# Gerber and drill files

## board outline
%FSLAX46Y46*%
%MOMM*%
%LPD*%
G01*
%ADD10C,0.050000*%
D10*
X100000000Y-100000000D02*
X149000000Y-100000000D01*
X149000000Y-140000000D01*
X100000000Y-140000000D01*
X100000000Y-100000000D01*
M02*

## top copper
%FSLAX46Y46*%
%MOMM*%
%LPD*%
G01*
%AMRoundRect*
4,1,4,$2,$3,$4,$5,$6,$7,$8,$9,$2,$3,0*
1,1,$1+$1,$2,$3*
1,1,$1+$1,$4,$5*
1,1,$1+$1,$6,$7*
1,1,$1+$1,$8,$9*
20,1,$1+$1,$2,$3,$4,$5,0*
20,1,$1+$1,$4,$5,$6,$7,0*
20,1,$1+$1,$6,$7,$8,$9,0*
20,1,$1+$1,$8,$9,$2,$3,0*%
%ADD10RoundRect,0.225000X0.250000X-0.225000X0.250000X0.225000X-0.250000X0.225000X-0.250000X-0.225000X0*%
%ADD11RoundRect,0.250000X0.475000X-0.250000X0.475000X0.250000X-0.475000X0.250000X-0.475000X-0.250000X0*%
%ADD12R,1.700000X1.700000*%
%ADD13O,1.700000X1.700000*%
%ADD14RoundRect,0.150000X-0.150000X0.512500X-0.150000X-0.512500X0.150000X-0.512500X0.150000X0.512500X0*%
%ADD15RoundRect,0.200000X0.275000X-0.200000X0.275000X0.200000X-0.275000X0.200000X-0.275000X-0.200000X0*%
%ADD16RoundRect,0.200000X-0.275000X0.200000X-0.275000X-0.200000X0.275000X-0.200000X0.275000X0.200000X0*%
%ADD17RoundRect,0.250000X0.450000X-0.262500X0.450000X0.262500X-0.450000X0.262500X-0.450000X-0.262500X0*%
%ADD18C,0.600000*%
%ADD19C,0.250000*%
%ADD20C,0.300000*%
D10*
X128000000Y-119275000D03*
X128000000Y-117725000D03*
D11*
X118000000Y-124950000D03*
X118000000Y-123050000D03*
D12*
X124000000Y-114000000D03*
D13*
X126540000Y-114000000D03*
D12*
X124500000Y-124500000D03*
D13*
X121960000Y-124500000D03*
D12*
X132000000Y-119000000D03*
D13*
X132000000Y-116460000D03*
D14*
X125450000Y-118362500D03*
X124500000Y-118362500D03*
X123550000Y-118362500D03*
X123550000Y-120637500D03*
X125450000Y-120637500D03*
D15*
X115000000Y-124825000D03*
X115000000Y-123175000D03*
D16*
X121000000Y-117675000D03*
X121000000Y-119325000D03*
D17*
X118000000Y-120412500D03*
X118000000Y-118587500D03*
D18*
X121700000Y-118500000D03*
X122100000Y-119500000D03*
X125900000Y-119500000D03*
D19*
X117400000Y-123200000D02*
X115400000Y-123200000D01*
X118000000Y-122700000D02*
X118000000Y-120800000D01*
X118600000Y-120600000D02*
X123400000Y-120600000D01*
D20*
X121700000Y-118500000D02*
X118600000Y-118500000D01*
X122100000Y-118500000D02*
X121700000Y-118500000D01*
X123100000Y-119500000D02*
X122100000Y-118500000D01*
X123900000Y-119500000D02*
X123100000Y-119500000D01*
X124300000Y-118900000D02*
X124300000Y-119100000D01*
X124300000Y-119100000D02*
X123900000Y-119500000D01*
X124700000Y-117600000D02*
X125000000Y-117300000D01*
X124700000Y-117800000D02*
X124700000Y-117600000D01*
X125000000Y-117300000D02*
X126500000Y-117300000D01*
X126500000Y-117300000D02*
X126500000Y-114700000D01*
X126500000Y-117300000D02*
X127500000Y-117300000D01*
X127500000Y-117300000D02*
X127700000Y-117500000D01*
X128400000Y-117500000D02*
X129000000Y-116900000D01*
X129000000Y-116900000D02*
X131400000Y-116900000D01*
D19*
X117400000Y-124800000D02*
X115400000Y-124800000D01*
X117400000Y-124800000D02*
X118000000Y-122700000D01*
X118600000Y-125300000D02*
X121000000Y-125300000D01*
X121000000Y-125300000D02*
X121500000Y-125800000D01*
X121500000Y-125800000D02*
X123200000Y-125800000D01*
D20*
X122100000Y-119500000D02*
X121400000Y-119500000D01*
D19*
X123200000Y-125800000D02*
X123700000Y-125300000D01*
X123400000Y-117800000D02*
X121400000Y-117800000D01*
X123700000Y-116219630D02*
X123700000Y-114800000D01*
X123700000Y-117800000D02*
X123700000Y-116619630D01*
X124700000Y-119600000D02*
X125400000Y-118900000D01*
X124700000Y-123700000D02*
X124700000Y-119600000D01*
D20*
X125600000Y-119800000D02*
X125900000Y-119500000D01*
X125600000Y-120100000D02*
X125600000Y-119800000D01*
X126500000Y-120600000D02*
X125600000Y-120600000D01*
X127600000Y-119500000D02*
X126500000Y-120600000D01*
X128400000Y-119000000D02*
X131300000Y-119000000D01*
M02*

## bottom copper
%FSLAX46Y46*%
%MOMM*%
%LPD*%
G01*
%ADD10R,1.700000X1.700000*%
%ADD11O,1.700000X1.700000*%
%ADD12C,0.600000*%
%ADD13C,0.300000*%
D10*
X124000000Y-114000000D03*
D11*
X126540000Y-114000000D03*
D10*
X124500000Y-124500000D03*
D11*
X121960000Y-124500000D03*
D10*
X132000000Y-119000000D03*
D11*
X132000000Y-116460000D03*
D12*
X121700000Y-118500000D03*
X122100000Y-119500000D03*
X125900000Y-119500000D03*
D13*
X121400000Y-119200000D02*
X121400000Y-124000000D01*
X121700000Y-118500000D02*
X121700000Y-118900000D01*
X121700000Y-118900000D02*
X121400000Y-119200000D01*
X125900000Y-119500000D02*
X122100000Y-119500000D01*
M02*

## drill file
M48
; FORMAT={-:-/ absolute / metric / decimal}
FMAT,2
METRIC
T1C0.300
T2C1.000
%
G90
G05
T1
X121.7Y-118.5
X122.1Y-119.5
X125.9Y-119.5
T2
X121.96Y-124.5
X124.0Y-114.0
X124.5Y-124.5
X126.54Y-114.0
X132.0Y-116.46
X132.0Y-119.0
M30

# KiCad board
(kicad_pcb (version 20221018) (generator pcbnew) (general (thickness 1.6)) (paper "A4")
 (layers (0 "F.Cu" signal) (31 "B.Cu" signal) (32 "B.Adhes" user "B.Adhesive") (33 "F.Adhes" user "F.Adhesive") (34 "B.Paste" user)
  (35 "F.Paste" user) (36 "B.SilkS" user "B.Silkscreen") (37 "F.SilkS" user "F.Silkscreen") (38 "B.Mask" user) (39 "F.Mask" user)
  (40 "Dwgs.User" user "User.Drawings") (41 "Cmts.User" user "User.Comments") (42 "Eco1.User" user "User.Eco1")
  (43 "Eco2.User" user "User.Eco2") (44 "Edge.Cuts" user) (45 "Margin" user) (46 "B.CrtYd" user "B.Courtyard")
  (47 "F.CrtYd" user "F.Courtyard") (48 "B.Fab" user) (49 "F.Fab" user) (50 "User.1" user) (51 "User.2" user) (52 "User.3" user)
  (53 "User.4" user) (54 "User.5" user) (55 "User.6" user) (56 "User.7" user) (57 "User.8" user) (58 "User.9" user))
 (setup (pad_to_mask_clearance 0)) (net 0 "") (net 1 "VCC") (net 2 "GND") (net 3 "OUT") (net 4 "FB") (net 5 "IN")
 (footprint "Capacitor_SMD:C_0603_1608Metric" (layer "F.Cu") (at 128 118.5 90)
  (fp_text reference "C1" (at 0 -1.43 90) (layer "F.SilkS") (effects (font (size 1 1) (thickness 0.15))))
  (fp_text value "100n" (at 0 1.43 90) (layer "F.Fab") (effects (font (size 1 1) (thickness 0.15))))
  (pad "1" smd roundrect (at -0.775 0 90) (size 0.9 0.95) (layers "F.Cu" "F.Paste" "F.Mask") (roundrect_rratio 0.25) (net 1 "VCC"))
  (pad "2" smd roundrect (at 0.775 0 90) (size 0.9 0.95) (layers "F.Cu" "F.Paste" "F.Mask") (roundrect_rratio 0.25) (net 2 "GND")))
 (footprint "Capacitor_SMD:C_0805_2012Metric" (layer "F.Cu") (at 118 124 90)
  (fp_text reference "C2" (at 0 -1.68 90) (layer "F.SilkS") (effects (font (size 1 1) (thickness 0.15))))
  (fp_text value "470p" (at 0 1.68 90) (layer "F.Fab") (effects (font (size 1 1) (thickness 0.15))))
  (pad "1" smd roundrect (at -0.95 0 90) (size 1 1.45) (layers "F.Cu" "F.Paste" "F.Mask") (roundrect_rratio 0.25) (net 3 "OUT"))
  (pad "2" smd roundrect (at 0.95 0 90) (size 1 1.45) (layers "F.Cu" "F.Paste" "F.Mask") (roundrect_rratio 0.25) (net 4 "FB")))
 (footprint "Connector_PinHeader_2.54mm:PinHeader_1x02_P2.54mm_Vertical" (layer "F.Cu") (at 124 114 90)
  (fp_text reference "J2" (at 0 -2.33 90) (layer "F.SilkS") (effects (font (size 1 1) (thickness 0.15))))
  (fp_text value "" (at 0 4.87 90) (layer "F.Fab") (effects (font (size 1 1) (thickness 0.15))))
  (pad "1" thru_hole rect (at 0 0 90) (size 1.7 1.7) (drill 1) (layers "*.Cu" "*.Mask") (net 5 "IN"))
  (pad "2" thru_hole oval (at 0 2.54 90) (size 1.7 1.7) (drill 1) (layers "*.Cu" "*.Mask") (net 2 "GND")))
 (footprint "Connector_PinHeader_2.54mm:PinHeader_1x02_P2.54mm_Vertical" (layer "F.Cu") (at 124.5 124.5 -90)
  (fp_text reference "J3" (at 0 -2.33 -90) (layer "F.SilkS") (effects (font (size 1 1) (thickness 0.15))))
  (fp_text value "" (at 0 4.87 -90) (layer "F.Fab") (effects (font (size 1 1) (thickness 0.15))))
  (pad "1" thru_hole rect (at 0 0 270) (size 1.7 1.7) (drill 1) (layers "*.Cu" "*.Mask") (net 3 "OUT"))
  (pad "2" thru_hole oval (at 0 2.54 270) (size 1.7 1.7) (drill 1) (layers "*.Cu" "*.Mask") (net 2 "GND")))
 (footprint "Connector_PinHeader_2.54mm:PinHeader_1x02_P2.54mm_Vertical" (layer "F.Cu") (at 132 119 180)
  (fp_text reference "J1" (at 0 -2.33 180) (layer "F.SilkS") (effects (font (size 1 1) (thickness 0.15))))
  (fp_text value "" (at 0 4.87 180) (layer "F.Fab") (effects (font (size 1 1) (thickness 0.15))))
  (pad "1" thru_hole rect (at 0 0 180) (size 1.7 1.7) (drill 1) (layers "*.Cu" "*.Mask") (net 1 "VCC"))
  (pad "2" thru_hole oval (at 0 2.54 180) (size 1.7 1.7) (drill 1) (layers "*.Cu" "*.Mask") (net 2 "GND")))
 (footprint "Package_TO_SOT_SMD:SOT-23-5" (layer "F.Cu") (at 124.5 119.5 -90)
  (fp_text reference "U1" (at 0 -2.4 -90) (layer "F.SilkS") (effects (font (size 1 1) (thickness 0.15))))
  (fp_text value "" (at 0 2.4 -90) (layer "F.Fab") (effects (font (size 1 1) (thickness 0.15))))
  (pad "1" smd roundrect (at -1.1375 -0.95 270) (size 1.325 0.6) (layers "F.Cu" "F.Paste" "F.Mask") (roundrect_rratio 0.25) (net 3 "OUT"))
  (pad "2" smd roundrect (at -1.1375 0 270) (size 1.325 0.6) (layers "F.Cu" "F.Paste" "F.Mask") (roundrect_rratio 0.25) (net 2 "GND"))
  (pad "3" smd roundrect (at -1.1375 0.95 270) (size 1.325 0.6) (layers "F.Cu" "F.Paste" "F.Mask") (roundrect_rratio 0.25) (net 5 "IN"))
  (pad "4" smd roundrect (at 1.1375 0.95 270) (size 1.325 0.6) (layers "F.Cu" "F.Paste" "F.Mask") (roundrect_rratio 0.25) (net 4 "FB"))
  (pad "5" smd roundrect (at 1.1375 -0.95 270) (size 1.325 0.6) (layers "F.Cu" "F.Paste" "F.Mask") (roundrect_rratio 0.25) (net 1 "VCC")))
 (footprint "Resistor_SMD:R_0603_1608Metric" (layer "F.Cu") (at 115 124 90)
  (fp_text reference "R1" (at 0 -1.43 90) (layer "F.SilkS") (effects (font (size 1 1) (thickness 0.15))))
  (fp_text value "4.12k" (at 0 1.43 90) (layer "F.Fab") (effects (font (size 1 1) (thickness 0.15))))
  (pad "1" smd roundrect (at -0.825 0 90) (size 0.8 0.95) (layers "F.Cu" "F.Paste" "F.Mask") (roundrect_rratio 0.25) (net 3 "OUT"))
  (pad "2" smd roundrect (at 0.825 0 90) (size 0.8 0.95) (layers "F.Cu" "F.Paste" "F.Mask") (roundrect_rratio 0.25) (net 4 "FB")))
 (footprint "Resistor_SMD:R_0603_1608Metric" (layer "F.Cu") (at 121 118.5 -90)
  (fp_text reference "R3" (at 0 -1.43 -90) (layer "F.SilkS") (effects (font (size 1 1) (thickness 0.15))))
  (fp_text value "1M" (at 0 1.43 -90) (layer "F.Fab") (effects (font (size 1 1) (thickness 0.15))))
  (pad "1" smd roundrect (at -0.825 0 270) (size 0.8 0.95) (layers "F.Cu" "F.Paste" "F.Mask") (roundrect_rratio 0.25) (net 5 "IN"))
  (pad "2" smd roundrect (at 0.825 0 270) (size 0.8 0.95) (layers "F.Cu" "F.Paste" "F.Mask") (roundrect_rratio 0.25) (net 1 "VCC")))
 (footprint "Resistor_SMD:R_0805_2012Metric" (layer "F.Cu") (at 118 119.5 90)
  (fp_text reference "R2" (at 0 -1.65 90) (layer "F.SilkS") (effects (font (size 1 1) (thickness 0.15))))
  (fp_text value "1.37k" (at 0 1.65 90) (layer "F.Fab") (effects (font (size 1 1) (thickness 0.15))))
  (pad "1" smd roundrect (at -0.9125 0 90) (size 1.025 1.4) (layers "F.Cu" "F.Paste" "F.Mask") (roundrect_rratio 0.243902) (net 4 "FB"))
  (pad "2" smd roundrect (at 0.9125 0 90) (size 1.025 1.4) (layers "F.Cu" "F.Paste" "F.Mask") (roundrect_rratio 0.243902) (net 2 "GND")))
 (gr_rect (start 100 100) (end 149 140) (stroke (width 0.05) (type default)) (fill none) (layer "Edge.Cuts"))
 (segment (start 117.4 123.2) (end 115.4 123.2) (width 0.25) (layer "F.Cu") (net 4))
 (segment (start 118 122.7) (end 118 120.8) (width 0.25) (layer "F.Cu") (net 4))
 (segment (start 118.6 120.6) (end 123.4 120.6) (width 0.25) (layer "F.Cu") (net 4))
 (segment (start 121.7 118.5) (end 118.6 118.5) (width 0.3) (layer "F.Cu") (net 2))
 (segment (start 122.1 118.5) (end 121.7 118.5) (width 0.3) (layer "F.Cu") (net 2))
 (segment (start 123.1 119.5) (end 122.1 118.5) (width 0.3) (layer "F.Cu") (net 2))
 (segment (start 123.9 119.5) (end 123.1 119.5) (width 0.3) (layer "F.Cu") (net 2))
 (segment (start 124.3 118.9) (end 124.3 119.1) (width 0.3) (layer "F.Cu") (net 2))
 (segment (start 124.3 119.1) (end 123.9 119.5) (width 0.3) (layer "F.Cu") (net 2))
 (segment (start 124.7 117.6) (end 125 117.3) (width 0.3) (layer "F.Cu") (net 2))
 (segment (start 124.7 117.8) (end 124.7 117.6) (width 0.3) (layer "F.Cu") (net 2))
 (segment (start 125 117.3) (end 126.5 117.3) (width 0.3) (layer "F.Cu") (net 2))
 (segment (start 126.5 117.3) (end 126.5 114.7) (width 0.3) (layer "F.Cu") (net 2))
 (segment (start 126.5 117.3) (end 127.5 117.3) (width 0.3) (layer "F.Cu") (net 2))
 (segment (start 127.5 117.3) (end 127.7 117.5) (width 0.3) (layer "F.Cu") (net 2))
 (segment (start 128.4 117.5) (end 129 116.9) (width 0.3) (layer "F.Cu") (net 2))
 (segment (start 129 116.9) (end 131.4 116.9) (width 0.3) (layer "F.Cu") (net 2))
 (via (at 121.7 118.5) (size 0.6) (drill 0.3) (layers "F.Cu" "B.Cu") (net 2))
 (segment (start 117.4 124.8) (end 115.4 124.8) (width 0.25) (layer "F.Cu") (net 3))
 (segment (start 117.4 124.8) (end 118 122.7) (width 0.25) (layer "F.Cu") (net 3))
 (segment (start 118.6 125.3) (end 121 125.3) (width 0.25) (layer "F.Cu") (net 3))
 (segment (start 121 125.3) (end 121.5 125.8) (width 0.25) (layer "F.Cu") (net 3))
 (segment (start 121.4 119.2) (end 121.4 124) (width 0.3) (layer "B.Cu") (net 2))
 (segment (start 121.5 125.8) (end 123.2 125.8) (width 0.25) (layer "F.Cu") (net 3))
 (segment (start 121.7 118.5) (end 121.7 118.9) (width 0.3) (layer "B.Cu") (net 2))
 (segment (start 121.7 118.9) (end 121.4 119.2) (width 0.3) (layer "B.Cu") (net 2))
 (segment (start 122.1 119.5) (end 121.4 119.5) (width 0.3) (layer "F.Cu") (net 1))
 (segment (start 123.2 125.8) (end 123.7 125.3) (width 0.25) (layer "F.Cu") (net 3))
 (segment (start 123.4 117.8) (end 121.4 117.8) (width 0.25) (layer "F.Cu") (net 5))
 (segment (start 123.7 116.21963) (end 123.7 114.8) (width 0.25) (layer "F.Cu") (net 5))
 (segment (start 123.7 117.8) (end 123.7 116.61963) (width 0.25) (layer "F.Cu") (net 5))
 (segment (start 124.7 119.6) (end 125.4 118.9) (width 0.25) (layer "F.Cu") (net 3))
 (segment (start 124.7 123.7) (end 124.7 119.6) (width 0.25) (layer "F.Cu") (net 3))
 (segment (start 125.6 119.8) (end 125.9 119.5) (width 0.3) (layer "F.Cu") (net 1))
 (segment (start 125.6 120.1) (end 125.6 119.8) (width 0.3) (layer "F.Cu") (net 1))
 (segment (start 126.5 120.6) (end 125.6 120.6) (width 0.3) (layer "F.Cu") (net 1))
 (segment (start 127.6 119.5) (end 126.5 120.6) (width 0.3) (layer "F.Cu") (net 1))
 (segment (start 128.4 119) (end 131.3 119) (width 0.3) (layer "F.Cu") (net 1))
 (via (at 122.1 119.5) (size 0.6) (drill 0.3) (layers "F.Cu" "B.Cu") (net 1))
 (via (at 125.9 119.5) (size 0.6) (drill 0.3) (layers "F.Cu" "B.Cu") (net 1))
 (segment (start 125.9 119.5) (end 122.1 119.5) (width 0.3) (layer "B.Cu") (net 1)))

